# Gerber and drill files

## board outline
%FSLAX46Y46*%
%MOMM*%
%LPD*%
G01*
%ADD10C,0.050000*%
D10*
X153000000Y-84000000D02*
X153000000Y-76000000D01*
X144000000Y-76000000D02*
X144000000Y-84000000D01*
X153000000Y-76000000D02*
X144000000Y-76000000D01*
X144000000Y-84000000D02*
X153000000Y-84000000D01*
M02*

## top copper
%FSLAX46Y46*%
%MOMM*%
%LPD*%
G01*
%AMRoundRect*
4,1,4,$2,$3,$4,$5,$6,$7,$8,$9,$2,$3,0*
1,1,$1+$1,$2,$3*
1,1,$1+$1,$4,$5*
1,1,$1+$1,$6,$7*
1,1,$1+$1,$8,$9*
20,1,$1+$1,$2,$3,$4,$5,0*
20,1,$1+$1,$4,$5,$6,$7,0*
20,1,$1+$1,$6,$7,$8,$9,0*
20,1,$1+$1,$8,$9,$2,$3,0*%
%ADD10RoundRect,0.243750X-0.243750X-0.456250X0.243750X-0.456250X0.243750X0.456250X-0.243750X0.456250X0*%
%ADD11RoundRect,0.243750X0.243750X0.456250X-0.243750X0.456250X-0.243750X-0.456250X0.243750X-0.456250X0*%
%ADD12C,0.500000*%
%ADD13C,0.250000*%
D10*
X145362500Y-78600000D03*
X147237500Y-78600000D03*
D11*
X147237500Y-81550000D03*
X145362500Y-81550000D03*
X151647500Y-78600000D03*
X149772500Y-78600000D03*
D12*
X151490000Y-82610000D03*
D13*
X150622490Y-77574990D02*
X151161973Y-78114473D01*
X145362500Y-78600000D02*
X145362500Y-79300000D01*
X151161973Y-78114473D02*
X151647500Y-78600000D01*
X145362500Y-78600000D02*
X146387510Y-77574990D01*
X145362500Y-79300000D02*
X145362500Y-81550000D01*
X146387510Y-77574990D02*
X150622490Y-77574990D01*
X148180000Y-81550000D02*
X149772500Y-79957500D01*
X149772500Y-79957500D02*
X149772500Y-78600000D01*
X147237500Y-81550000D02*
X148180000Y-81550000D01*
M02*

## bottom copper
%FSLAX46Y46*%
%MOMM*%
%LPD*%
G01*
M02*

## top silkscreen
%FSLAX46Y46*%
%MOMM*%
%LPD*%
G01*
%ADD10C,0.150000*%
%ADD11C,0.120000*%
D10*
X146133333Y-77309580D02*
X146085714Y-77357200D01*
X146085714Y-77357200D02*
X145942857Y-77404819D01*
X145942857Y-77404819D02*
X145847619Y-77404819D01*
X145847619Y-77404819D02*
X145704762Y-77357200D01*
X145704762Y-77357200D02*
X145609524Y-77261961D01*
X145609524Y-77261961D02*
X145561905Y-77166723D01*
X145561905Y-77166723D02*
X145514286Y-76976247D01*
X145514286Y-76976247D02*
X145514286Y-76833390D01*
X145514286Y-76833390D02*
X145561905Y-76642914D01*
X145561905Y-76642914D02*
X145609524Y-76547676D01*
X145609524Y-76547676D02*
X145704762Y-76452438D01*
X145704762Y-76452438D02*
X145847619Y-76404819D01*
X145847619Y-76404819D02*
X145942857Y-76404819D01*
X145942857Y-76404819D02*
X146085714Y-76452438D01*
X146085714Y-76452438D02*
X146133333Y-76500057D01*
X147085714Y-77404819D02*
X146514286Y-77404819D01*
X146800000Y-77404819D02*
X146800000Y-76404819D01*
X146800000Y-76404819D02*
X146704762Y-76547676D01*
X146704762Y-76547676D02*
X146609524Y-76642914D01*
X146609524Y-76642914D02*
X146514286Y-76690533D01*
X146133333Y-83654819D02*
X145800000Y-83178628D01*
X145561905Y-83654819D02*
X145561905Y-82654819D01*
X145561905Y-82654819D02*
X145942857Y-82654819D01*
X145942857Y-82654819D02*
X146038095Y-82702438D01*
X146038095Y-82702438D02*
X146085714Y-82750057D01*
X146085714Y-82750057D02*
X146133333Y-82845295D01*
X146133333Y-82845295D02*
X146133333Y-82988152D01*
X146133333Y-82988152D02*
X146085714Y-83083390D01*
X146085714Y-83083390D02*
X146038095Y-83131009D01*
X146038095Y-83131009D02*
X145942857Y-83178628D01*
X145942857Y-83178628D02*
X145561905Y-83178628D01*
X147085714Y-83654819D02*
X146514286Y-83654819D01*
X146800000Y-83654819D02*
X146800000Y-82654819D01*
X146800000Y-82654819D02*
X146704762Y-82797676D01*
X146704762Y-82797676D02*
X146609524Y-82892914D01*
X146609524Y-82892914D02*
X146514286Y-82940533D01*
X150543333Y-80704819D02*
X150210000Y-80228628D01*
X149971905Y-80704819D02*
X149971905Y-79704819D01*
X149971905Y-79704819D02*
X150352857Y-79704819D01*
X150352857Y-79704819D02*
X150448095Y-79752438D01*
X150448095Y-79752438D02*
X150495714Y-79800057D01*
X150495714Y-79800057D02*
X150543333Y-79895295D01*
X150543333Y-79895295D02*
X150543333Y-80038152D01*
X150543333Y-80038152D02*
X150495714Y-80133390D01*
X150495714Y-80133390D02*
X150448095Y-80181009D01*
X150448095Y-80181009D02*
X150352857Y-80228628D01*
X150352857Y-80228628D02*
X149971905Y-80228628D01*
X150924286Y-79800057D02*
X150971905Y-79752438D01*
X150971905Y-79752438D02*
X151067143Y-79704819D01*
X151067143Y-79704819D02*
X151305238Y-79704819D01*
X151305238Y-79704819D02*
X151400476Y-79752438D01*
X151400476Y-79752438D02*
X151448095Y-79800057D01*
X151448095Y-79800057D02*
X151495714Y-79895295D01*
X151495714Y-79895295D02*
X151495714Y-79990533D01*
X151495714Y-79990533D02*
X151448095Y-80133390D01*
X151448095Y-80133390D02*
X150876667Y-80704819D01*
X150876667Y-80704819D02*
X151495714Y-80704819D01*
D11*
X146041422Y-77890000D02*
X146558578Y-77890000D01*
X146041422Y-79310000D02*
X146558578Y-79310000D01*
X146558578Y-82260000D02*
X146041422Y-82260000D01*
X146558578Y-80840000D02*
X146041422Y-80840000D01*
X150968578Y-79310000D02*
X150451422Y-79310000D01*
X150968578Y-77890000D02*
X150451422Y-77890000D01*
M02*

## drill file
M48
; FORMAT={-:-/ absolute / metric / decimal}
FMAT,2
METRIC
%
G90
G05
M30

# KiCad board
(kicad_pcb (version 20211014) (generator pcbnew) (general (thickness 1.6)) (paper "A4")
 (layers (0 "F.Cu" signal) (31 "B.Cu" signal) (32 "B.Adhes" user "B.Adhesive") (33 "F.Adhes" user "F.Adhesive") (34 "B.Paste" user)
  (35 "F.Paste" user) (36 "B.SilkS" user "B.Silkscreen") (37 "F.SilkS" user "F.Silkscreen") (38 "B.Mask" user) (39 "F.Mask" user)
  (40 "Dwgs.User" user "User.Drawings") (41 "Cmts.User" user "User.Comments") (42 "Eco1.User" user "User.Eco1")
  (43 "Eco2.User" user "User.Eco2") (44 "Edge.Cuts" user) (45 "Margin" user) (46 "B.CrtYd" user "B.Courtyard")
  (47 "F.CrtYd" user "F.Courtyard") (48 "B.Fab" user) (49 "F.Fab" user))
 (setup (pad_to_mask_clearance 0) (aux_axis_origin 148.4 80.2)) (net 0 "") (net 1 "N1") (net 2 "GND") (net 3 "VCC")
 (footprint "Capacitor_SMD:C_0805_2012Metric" (layer "F.Cu") (at 146.3 78.6)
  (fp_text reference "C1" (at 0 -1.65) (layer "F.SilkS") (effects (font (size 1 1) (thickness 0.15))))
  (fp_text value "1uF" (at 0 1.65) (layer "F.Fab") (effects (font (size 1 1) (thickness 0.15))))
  (fp_line (start -0.258578 -0.71) (end 0.258578 -0.71) (layer "F.SilkS") (width 0.12))
  (fp_line (start -0.258578 0.71) (end 0.258578 0.71) (layer "F.SilkS") (width 0.12))
  (pad "1" smd roundrect locked (at -0.9375 0) (size 0.975 1.4) (layers "F.Cu" "F.Paste" "F.Mask") (roundrect_rratio 0.25) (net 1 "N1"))
  (pad "2" smd roundrect locked (at 0.9375 0) (size 0.975 1.4) (layers "F.Cu" "F.Paste" "F.Mask") (roundrect_rratio 0.25) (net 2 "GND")))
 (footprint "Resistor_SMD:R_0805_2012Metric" (layer "F.Cu") (at 146.3 81.55 180)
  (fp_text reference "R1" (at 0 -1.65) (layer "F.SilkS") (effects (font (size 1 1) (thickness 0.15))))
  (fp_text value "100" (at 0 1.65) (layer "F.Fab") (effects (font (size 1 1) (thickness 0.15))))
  (fp_line (start -0.258578 -0.71) (end 0.258578 -0.71) (layer "F.SilkS") (width 0.12))
  (fp_line (start -0.258578 0.71) (end 0.258578 0.71) (layer "F.SilkS") (width 0.12))
  (pad "1" smd roundrect locked (at -0.9375 0 180) (size 0.975 1.4) (layers "F.Cu" "F.Paste" "F.Mask") (roundrect_rratio 0.25) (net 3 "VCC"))
  (pad "2" smd roundrect locked (at 0.9375 0 180) (size 0.975 1.4) (layers "F.Cu" "F.Paste" "F.Mask") (roundrect_rratio 0.25) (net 1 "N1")))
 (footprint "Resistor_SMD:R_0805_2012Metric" (layer "F.Cu") (at 150.71 78.6 180)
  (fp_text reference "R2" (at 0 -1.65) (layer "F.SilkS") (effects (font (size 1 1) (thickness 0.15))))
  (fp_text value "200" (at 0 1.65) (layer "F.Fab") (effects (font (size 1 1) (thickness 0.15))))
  (fp_line (start -0.258578 -0.71) (end 0.258578 -0.71) (layer "F.SilkS") (width 0.12))
  (fp_line (start -0.258578 0.71) (end 0.258578 0.71) (layer "F.SilkS") (width 0.12))
  (pad "1" smd roundrect locked (at -0.9375 0 180) (size 0.975 1.4) (layers "F.Cu" "F.Paste" "F.Mask") (roundrect_rratio 0.25) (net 1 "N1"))
  (pad "2" smd roundrect locked (at 0.9375 0 180) (size 0.975 1.4) (layers "F.Cu" "F.Paste" "F.Mask") (roundrect_rratio 0.25) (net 3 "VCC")))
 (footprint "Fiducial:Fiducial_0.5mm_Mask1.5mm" (layer "F.Cu") (at 151.49 82.61)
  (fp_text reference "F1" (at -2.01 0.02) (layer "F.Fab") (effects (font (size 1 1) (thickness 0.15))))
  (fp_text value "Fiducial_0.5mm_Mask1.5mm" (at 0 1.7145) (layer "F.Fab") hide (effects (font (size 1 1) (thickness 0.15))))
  (pad "" smd circle (at 0 0) (size 0.5 0.5) (layers "F.Cu" "F.Mask") (solder_mask_margin 0.5) (clearance 0.5)))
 (gr_line (start 153 84) (end 153 76) (layer "Edge.Cuts") (width 0.05))
 (gr_line (start 144 76) (end 144 84) (layer "Edge.Cuts") (width 0.05))
 (gr_line (start 153 76) (end 144 76) (layer "Edge.Cuts") (width 0.05))
 (gr_line (start 144 84) (end 153 84) (layer "Edge.Cuts") (width 0.05))
 (segment (start 150.62249 77.57499) (end 151.161973 78.114473) (width 0.25) (layer "F.Cu") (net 1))
 (segment (start 145.3625 78.6) (end 145.3625 79.3) (width 0.25) (layer "F.Cu") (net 1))
 (segment (start 151.161973 78.114473) (end 151.6475 78.6) (width 0.25) (layer "F.Cu") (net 1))
 (segment (start 145.3625 78.6) (end 146.38751 77.57499) (width 0.25) (layer "F.Cu") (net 1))
 (segment (start 145.3625 79.3) (end 145.3625 81.55) (width 0.25) (layer "F.Cu") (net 1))
 (segment (start 146.38751 77.57499) (end 150.62249 77.57499) (width 0.25) (layer "F.Cu") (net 1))
 (segment (start 148.18 81.55) (end 149.7725 79.9575) (width 0.25) (layer "F.Cu") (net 3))
 (segment (start 149.7725 79.9575) (end 149.7725 78.6) (width 0.25) (layer "F.Cu") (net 3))
 (segment (start 147.2375 81.55) (end 148.18 81.55) (width 0.25) (layer "F.Cu") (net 3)))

